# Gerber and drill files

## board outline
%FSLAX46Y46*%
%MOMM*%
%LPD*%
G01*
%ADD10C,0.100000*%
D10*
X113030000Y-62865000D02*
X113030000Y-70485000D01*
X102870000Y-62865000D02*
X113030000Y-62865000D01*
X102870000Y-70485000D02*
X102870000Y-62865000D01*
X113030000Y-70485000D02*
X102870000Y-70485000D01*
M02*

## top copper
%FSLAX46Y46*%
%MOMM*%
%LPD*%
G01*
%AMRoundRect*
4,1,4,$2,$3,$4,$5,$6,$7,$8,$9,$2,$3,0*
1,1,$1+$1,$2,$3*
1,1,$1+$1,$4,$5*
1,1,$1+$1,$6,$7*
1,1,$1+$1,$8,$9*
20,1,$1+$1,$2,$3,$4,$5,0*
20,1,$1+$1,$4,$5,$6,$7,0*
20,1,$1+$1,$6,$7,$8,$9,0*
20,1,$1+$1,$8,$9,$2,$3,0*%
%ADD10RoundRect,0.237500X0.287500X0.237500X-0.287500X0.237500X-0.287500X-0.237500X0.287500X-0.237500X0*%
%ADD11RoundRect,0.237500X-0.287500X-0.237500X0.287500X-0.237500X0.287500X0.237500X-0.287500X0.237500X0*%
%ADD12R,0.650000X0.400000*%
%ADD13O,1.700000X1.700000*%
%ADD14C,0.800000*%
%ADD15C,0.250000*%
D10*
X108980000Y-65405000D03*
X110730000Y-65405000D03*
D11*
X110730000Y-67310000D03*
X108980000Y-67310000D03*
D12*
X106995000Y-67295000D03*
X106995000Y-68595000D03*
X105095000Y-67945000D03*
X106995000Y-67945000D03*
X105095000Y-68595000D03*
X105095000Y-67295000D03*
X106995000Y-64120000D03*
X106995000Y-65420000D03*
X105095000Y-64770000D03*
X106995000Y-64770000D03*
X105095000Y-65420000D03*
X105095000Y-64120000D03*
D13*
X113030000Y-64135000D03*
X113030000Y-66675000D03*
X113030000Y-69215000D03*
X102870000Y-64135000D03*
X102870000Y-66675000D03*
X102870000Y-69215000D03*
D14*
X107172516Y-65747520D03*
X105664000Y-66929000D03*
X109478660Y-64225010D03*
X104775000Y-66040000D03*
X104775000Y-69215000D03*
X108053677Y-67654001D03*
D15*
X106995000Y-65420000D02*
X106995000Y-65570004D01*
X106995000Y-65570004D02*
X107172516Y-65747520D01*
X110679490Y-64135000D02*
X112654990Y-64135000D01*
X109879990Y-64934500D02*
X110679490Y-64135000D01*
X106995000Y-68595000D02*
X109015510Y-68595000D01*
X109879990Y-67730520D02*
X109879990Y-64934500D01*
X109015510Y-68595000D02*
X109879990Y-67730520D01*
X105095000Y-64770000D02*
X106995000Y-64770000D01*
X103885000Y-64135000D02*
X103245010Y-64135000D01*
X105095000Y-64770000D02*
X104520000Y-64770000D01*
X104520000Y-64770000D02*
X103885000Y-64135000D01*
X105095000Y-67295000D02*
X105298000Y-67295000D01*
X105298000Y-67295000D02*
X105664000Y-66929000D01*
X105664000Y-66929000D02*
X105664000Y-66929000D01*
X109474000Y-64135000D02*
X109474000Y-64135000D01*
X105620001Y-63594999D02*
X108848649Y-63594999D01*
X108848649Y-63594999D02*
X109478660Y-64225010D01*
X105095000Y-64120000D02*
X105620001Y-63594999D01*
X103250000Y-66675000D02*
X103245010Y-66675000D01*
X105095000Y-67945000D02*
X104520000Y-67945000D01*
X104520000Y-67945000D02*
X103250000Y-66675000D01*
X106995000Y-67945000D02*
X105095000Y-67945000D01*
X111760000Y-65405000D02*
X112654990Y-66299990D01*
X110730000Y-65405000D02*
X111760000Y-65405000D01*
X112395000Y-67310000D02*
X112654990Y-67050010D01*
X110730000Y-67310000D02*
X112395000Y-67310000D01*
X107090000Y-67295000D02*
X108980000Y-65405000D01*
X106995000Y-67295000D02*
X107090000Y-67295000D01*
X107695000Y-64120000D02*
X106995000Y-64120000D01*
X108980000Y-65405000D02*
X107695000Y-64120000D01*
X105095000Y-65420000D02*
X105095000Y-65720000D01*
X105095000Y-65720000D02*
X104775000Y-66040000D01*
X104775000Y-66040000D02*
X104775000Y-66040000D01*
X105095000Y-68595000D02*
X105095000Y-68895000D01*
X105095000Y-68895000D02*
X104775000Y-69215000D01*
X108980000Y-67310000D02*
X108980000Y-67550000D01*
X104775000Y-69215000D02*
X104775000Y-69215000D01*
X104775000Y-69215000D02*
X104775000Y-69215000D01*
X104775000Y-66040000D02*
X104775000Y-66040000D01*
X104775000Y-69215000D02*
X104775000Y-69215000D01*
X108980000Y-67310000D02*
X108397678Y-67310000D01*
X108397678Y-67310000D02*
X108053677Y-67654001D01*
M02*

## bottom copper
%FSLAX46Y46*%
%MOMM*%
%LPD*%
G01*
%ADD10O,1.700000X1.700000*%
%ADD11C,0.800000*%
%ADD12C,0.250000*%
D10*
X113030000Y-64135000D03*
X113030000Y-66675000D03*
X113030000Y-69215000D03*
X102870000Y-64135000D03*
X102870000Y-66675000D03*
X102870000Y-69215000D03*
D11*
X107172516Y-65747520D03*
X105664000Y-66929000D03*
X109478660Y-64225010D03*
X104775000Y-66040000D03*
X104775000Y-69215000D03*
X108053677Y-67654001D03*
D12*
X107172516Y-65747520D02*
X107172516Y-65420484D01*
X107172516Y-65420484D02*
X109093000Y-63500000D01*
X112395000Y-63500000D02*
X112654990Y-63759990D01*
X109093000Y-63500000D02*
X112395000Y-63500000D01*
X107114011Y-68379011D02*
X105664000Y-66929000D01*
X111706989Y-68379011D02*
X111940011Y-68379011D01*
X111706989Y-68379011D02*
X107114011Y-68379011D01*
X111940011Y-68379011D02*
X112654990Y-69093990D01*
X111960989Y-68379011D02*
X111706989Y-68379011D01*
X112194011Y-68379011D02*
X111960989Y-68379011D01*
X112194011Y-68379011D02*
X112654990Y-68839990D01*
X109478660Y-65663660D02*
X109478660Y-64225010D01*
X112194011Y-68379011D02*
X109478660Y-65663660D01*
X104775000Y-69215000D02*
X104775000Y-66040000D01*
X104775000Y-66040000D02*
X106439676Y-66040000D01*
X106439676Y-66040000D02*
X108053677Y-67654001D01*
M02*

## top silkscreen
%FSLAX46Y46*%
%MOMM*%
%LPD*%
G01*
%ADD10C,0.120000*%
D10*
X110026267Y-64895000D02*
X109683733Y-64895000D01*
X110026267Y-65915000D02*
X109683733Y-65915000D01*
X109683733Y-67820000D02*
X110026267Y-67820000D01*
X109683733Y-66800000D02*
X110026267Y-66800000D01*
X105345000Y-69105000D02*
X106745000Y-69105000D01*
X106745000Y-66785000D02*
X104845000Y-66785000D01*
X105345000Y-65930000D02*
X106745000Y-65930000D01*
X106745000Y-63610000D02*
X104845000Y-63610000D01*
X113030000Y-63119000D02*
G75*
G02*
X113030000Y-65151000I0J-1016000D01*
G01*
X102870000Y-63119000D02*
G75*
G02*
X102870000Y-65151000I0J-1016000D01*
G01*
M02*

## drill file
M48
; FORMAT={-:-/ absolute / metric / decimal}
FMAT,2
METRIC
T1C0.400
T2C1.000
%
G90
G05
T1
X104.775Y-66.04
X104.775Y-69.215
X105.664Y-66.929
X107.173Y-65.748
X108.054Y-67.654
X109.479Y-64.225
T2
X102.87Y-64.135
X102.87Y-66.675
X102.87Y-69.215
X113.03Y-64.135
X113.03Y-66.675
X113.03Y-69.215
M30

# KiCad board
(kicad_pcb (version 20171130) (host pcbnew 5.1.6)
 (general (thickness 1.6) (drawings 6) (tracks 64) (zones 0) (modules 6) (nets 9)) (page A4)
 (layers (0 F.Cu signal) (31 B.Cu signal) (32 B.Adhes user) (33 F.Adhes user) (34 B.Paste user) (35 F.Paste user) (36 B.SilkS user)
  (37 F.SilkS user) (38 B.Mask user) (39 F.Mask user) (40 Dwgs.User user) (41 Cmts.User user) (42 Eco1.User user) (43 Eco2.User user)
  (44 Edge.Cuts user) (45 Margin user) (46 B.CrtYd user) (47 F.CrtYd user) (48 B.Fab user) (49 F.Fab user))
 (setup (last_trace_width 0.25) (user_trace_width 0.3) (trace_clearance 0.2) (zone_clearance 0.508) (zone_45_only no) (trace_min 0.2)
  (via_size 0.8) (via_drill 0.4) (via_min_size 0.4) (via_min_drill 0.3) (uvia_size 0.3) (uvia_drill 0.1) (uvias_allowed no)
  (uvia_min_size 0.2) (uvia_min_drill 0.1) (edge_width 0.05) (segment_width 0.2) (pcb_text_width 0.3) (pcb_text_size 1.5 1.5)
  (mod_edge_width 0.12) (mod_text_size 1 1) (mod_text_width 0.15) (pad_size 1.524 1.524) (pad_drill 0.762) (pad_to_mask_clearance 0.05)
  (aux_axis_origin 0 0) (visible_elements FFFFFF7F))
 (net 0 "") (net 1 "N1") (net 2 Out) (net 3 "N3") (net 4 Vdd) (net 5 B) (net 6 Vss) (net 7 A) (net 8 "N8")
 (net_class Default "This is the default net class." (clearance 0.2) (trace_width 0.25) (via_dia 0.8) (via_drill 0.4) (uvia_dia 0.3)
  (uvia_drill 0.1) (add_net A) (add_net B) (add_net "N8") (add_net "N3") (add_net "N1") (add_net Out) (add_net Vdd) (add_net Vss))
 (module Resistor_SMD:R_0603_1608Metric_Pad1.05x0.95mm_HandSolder (layer F.Cu) (at 109.855 65.405 180)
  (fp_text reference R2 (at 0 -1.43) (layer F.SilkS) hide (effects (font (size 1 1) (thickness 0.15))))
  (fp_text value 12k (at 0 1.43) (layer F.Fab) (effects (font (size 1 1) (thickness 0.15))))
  (fp_line (start -0.171267 0.51) (end 0.171267 0.51) (layer F.SilkS) (width 0.12))
  (fp_line (start -0.171267 -0.51) (end 0.171267 -0.51) (layer F.SilkS) (width 0.12))
  (pad 2 smd roundrect (at 0.875 0 180) (size 1.05 0.95) (layers F.Cu F.Paste F.Mask) (roundrect_rratio 0.25) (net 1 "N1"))
  (pad 1 smd roundrect (at -0.875 0 180) (size 1.05 0.95) (layers F.Cu F.Paste F.Mask) (roundrect_rratio 0.25) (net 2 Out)))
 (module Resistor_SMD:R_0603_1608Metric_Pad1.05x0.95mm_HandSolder (layer F.Cu) (at 109.855 67.31)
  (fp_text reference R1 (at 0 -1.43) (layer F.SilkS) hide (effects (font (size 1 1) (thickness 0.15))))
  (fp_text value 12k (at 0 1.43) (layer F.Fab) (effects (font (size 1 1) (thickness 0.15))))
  (fp_line (start -0.171267 0.51) (end 0.171267 0.51) (layer F.SilkS) (width 0.12))
  (fp_line (start -0.171267 -0.51) (end 0.171267 -0.51) (layer F.SilkS) (width 0.12))
  (pad 2 smd roundrect (at 0.875 0) (size 1.05 0.95) (layers F.Cu F.Paste F.Mask) (roundrect_rratio 0.25) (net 2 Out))
  (pad 1 smd roundrect (at -0.875 0) (size 1.05 0.95) (layers F.Cu F.Paste F.Mask) (roundrect_rratio 0.25) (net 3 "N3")))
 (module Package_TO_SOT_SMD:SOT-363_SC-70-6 (layer F.Cu) (at 106.045 67.945)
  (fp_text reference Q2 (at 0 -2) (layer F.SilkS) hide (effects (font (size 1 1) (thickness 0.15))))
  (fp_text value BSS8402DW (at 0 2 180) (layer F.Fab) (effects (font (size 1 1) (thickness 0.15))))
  (fp_line (start -0.7 1.16) (end 0.7 1.16) (layer F.SilkS) (width 0.12))
  (fp_line (start 0.7 -1.16) (end -1.2 -1.16) (layer F.SilkS) (width 0.12))
  (pad 6 smd rect (at 0.95 -0.65) (size 0.65 0.4) (layers F.Cu F.Paste F.Mask) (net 1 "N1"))
  (pad 4 smd rect (at 0.95 0.65) (size 0.65 0.4) (layers F.Cu F.Paste F.Mask) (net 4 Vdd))
  (pad 2 smd rect (at -0.95 0) (size 0.65 0.4) (layers F.Cu F.Paste F.Mask) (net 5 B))
  (pad 5 smd rect (at 0.95 0) (size 0.65 0.4) (layers F.Cu F.Paste F.Mask) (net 5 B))
  (pad 3 smd rect (at -0.95 0.65) (size 0.65 0.4) (layers F.Cu F.Paste F.Mask) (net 3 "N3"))
  (pad 1 smd rect (at -0.95 -0.65) (size 0.65 0.4) (layers F.Cu F.Paste F.Mask) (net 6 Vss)))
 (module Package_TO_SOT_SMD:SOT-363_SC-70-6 (layer F.Cu) (at 106.045 64.77)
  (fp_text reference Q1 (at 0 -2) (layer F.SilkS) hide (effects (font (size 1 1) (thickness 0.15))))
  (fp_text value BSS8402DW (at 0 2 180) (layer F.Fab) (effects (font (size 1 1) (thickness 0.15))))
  (fp_line (start -0.7 1.16) (end 0.7 1.16) (layer F.SilkS) (width 0.12))
  (fp_line (start 0.7 -1.16) (end -1.2 -1.16) (layer F.SilkS) (width 0.12))
  (pad 6 smd rect (at 0.95 -0.65) (size 0.65 0.4) (layers F.Cu F.Paste F.Mask) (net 1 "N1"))
  (pad 4 smd rect (at 0.95 0.65) (size 0.65 0.4) (layers F.Cu F.Paste F.Mask) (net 4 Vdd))
  (pad 2 smd rect (at -0.95 0) (size 0.65 0.4) (layers F.Cu F.Paste F.Mask) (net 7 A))
  (pad 5 smd rect (at 0.95 0) (size 0.65 0.4) (layers F.Cu F.Paste F.Mask) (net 7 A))
  (pad 3 smd rect (at -0.95 0.65) (size 0.65 0.4) (layers F.Cu F.Paste F.Mask) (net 3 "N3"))
  (pad 1 smd rect (at -0.95 -0.65) (size 0.65 0.4) (layers F.Cu F.Paste F.Mask) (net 6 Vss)))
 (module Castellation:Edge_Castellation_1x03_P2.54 (layer F.Cu) (at 113.03 64.135)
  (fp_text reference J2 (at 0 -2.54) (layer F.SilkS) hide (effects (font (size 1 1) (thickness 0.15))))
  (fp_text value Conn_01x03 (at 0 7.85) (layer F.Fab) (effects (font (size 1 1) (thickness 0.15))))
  (fp_arc (start 0 0) (end 0 1.016) (angle -180) (layer F.SilkS) (width 0.12))
  (pad 1 thru_hole oval (at 0 0) (size 1.7 1.7) (drill 1) (layers *.Cu *.Mask) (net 4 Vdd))
  (pad 2 thru_hole oval (at 0 2.54) (size 1.7 1.7) (drill 1) (layers *.Cu *.Mask) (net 2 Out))
  (pad 3 thru_hole oval (at 0 5.08) (size 1.7 1.7) (drill 1) (layers *.Cu *.Mask) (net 6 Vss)))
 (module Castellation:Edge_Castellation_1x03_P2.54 (layer F.Cu) (at 102.87 64.135)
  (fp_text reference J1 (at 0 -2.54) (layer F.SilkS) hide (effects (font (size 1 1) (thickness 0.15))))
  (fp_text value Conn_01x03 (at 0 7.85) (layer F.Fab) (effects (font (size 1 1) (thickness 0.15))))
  (fp_arc (start 0 0) (end 0 1.016) (angle -180) (layer F.SilkS) (width 0.12))
  (pad 1 thru_hole oval (at 0 0) (size 1.7 1.7) (drill 1) (layers *.Cu *.Mask) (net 7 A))
  (pad 2 thru_hole oval (at 0 2.54) (size 1.7 1.7) (drill 1) (layers *.Cu *.Mask) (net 5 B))
  (pad 3 thru_hole oval (at 0 5.08) (size 1.7 1.7) (drill 1) (layers *.Cu *.Mask) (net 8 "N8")))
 (gr_line (start 113.03 62.865) (end 113.03 70.485) (layer Edge.Cuts) (width 0.1))
 (gr_line (start 102.87 62.865) (end 113.03 62.865) (layer Edge.Cuts) (width 0.1))
 (gr_line (start 102.87 70.485) (end 102.87 62.865) (layer Edge.Cuts) (width 0.1))
 (gr_line (start 113.03 70.485) (end 102.87 70.485) (layer Edge.Cuts) (width 0.1))
 (segment (start 106.995 65.42) (end 106.995 65.570004) (width 0.25) (layer F.Cu) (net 4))
 (via (at 107.172516 65.74752) (size 0.8) (drill 0.4) (layers F.Cu B.Cu) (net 4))
 (segment (start 106.995 65.570004) (end 107.172516 65.74752) (width 0.25) (layer F.Cu) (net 4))
 (segment (start 110.67949 64.135) (end 112.65499 64.135) (width 0.25) (layer F.Cu) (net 4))
 (segment (start 109.87999 64.9345) (end 110.67949 64.135) (width 0.25) (layer F.Cu) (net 4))
 (segment (start 106.995 68.595) (end 109.01551 68.595) (width 0.25) (layer F.Cu) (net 4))
 (segment (start 109.87999 67.73052) (end 109.87999 64.9345) (width 0.25) (layer F.Cu) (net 4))
 (segment (start 109.01551 68.595) (end 109.87999 67.73052) (width 0.25) (layer F.Cu) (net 4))
 (segment (start 107.172516 65.74752) (end 107.172516 65.420484) (width 0.25) (layer B.Cu) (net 4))
 (segment (start 107.172516 65.420484) (end 109.093 63.5) (width 0.25) (layer B.Cu) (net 4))
 (segment (start 112.395 63.5) (end 112.65499 63.75999) (width 0.25) (layer B.Cu) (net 4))
 (segment (start 109.093 63.5) (end 112.395 63.5) (width 0.25) (layer B.Cu) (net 4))
 (segment (start 105.095 64.77) (end 106.995 64.77) (width 0.25) (layer F.Cu) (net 7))
 (segment (start 103.885 64.135) (end 103.24501 64.135) (width 0.25) (layer F.Cu) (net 7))
 (segment (start 105.095 64.77) (end 104.52 64.77) (width 0.25) (layer F.Cu) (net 7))
 (segment (start 104.52 64.77) (end 103.885 64.135) (width 0.25) (layer F.Cu) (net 7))
 (segment (start 105.095 67.295) (end 105.298 67.295) (width 0.25) (layer F.Cu) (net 6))
 (segment (start 105.298 67.295) (end 105.664 66.929) (width 0.25) (layer F.Cu) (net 6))
 (segment (start 105.664 66.929) (end 105.664 66.929) (width 0.25) (layer F.Cu) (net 6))
 (via (at 105.664 66.929) (size 0.8) (drill 0.4) (layers F.Cu B.Cu) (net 6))
 (segment (start 107.114011 68.379011) (end 105.664 66.929) (width 0.25) (layer B.Cu) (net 6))
 (segment (start 111.706989 68.379011) (end 111.940011 68.379011) (width 0.25) (layer B.Cu) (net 6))
 (segment (start 111.706989 68.379011) (end 107.114011 68.379011) (width 0.25) (layer B.Cu) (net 6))
 (segment (start 111.940011 68.379011) (end 112.65499 69.09399) (width 0.25) (layer B.Cu) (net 6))
 (segment (start 109.474 64.135) (end 109.474 64.135) (width 0.25) (layer F.Cu) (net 6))
 (segment (start 111.960989 68.379011) (end 111.706989 68.379011) (width 0.25) (layer B.Cu) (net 6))
 (segment (start 112.194011 68.379011) (end 111.960989 68.379011) (width 0.25) (layer B.Cu) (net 6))
 (segment (start 112.194011 68.379011) (end 112.65499 68.83999) (width 0.25) (layer B.Cu) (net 6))
 (segment (start 105.620001 63.594999) (end 108.848649 63.594999) (width 0.25) (layer F.Cu) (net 6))
 (segment (start 108.848649 63.594999) (end 109.47866 64.22501) (width 0.25) (layer F.Cu) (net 6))
 (segment (start 109.47866 65.66366) (end 109.47866 64.22501) (width 0.25) (layer B.Cu) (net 6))
 (segment (start 112.194011 68.379011) (end 109.47866 65.66366) (width 0.25) (layer B.Cu) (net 6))
 (via (at 109.47866 64.22501) (size 0.8) (drill 0.4) (layers F.Cu B.Cu) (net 6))
 (segment (start 105.095 64.12) (end 105.620001 63.594999) (width 0.25) (layer F.Cu) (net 6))
 (segment (start 103.25 66.675) (end 103.24501 66.675) (width 0.25) (layer F.Cu) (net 5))
 (segment (start 105.095 67.945) (end 104.52 67.945) (width 0.25) (layer F.Cu) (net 5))
 (segment (start 104.52 67.945) (end 103.25 66.675) (width 0.25) (layer F.Cu) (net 5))
 (segment (start 106.995 67.945) (end 105.095 67.945) (width 0.25) (layer F.Cu) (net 5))
 (segment (start 111.76 65.405) (end 112.65499 66.29999) (width 0.25) (layer F.Cu) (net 2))
 (segment (start 110.73 65.405) (end 111.76 65.405) (width 0.25) (layer F.Cu) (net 2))
 (segment (start 112.395 67.31) (end 112.65499 67.05001) (width 0.25) (layer F.Cu) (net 2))
 (segment (start 110.73 67.31) (end 112.395 67.31) (width 0.25) (layer F.Cu) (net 2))
 (segment (start 107.09 67.295) (end 108.98 65.405) (width 0.25) (layer F.Cu) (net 1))
 (segment (start 106.995 67.295) (end 107.09 67.295) (width 0.25) (layer F.Cu) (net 1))
 (segment (start 107.695 64.12) (end 106.995 64.12) (width 0.25) (layer F.Cu) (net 1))
 (segment (start 108.98 65.405) (end 107.695 64.12) (width 0.25) (layer F.Cu) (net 1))
 (segment (start 105.095 65.42) (end 105.095 65.72) (width 0.25) (layer F.Cu) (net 3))
 (segment (start 105.095 65.72) (end 104.775 66.04) (width 0.25) (layer F.Cu) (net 3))
 (segment (start 104.775 66.04) (end 104.775 66.04) (width 0.25) (layer F.Cu) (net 3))
 (segment (start 105.095 68.595) (end 105.095 68.895) (width 0.25) (layer F.Cu) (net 3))
 (segment (start 105.095 68.895) (end 104.775 69.215) (width 0.25) (layer F.Cu) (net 3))
 (segment (start 108.98 67.31) (end 108.98 67.55) (width 0.25) (layer F.Cu) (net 3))
 (segment (start 104.775 69.215) (end 104.775 69.215) (width 0.25) (layer F.Cu) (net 3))
 (segment (start 104.775 69.215) (end 104.775 69.215) (width 0.25) (layer F.Cu) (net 3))
 (segment (start 104.775 66.04) (end 104.775 66.04) (width 0.25) (layer F.Cu) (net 3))
 (via (at 104.775 66.04) (size 0.8) (drill 0.4) (layers F.Cu B.Cu) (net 3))
 (segment (start 104.775 69.215) (end 104.775 69.215) (width 0.25) (layer F.Cu) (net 3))
 (via (at 104.775 69.215) (size 0.8) (drill 0.4) (layers F.Cu B.Cu) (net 3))
 (segment (start 104.775 69.215) (end 104.775 66.04) (width 0.25) (layer B.Cu) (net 3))
 (segment (start 108.98 67.31) (end 108.397678 67.31) (width 0.25) (layer F.Cu) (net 3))
 (segment (start 104.775 66.04) (end 106.439676 66.04) (width 0.25) (layer B.Cu) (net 3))
 (segment (start 106.439676 66.04) (end 108.053677 67.654001) (width 0.25) (layer B.Cu) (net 3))
 (via (at 108.053677 67.654001) (size 0.8) (drill 0.4) (layers F.Cu B.Cu) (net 3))
 (segment (start 108.397678 67.31) (end 108.053677 67.654001) (width 0.25) (layer F.Cu) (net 3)))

